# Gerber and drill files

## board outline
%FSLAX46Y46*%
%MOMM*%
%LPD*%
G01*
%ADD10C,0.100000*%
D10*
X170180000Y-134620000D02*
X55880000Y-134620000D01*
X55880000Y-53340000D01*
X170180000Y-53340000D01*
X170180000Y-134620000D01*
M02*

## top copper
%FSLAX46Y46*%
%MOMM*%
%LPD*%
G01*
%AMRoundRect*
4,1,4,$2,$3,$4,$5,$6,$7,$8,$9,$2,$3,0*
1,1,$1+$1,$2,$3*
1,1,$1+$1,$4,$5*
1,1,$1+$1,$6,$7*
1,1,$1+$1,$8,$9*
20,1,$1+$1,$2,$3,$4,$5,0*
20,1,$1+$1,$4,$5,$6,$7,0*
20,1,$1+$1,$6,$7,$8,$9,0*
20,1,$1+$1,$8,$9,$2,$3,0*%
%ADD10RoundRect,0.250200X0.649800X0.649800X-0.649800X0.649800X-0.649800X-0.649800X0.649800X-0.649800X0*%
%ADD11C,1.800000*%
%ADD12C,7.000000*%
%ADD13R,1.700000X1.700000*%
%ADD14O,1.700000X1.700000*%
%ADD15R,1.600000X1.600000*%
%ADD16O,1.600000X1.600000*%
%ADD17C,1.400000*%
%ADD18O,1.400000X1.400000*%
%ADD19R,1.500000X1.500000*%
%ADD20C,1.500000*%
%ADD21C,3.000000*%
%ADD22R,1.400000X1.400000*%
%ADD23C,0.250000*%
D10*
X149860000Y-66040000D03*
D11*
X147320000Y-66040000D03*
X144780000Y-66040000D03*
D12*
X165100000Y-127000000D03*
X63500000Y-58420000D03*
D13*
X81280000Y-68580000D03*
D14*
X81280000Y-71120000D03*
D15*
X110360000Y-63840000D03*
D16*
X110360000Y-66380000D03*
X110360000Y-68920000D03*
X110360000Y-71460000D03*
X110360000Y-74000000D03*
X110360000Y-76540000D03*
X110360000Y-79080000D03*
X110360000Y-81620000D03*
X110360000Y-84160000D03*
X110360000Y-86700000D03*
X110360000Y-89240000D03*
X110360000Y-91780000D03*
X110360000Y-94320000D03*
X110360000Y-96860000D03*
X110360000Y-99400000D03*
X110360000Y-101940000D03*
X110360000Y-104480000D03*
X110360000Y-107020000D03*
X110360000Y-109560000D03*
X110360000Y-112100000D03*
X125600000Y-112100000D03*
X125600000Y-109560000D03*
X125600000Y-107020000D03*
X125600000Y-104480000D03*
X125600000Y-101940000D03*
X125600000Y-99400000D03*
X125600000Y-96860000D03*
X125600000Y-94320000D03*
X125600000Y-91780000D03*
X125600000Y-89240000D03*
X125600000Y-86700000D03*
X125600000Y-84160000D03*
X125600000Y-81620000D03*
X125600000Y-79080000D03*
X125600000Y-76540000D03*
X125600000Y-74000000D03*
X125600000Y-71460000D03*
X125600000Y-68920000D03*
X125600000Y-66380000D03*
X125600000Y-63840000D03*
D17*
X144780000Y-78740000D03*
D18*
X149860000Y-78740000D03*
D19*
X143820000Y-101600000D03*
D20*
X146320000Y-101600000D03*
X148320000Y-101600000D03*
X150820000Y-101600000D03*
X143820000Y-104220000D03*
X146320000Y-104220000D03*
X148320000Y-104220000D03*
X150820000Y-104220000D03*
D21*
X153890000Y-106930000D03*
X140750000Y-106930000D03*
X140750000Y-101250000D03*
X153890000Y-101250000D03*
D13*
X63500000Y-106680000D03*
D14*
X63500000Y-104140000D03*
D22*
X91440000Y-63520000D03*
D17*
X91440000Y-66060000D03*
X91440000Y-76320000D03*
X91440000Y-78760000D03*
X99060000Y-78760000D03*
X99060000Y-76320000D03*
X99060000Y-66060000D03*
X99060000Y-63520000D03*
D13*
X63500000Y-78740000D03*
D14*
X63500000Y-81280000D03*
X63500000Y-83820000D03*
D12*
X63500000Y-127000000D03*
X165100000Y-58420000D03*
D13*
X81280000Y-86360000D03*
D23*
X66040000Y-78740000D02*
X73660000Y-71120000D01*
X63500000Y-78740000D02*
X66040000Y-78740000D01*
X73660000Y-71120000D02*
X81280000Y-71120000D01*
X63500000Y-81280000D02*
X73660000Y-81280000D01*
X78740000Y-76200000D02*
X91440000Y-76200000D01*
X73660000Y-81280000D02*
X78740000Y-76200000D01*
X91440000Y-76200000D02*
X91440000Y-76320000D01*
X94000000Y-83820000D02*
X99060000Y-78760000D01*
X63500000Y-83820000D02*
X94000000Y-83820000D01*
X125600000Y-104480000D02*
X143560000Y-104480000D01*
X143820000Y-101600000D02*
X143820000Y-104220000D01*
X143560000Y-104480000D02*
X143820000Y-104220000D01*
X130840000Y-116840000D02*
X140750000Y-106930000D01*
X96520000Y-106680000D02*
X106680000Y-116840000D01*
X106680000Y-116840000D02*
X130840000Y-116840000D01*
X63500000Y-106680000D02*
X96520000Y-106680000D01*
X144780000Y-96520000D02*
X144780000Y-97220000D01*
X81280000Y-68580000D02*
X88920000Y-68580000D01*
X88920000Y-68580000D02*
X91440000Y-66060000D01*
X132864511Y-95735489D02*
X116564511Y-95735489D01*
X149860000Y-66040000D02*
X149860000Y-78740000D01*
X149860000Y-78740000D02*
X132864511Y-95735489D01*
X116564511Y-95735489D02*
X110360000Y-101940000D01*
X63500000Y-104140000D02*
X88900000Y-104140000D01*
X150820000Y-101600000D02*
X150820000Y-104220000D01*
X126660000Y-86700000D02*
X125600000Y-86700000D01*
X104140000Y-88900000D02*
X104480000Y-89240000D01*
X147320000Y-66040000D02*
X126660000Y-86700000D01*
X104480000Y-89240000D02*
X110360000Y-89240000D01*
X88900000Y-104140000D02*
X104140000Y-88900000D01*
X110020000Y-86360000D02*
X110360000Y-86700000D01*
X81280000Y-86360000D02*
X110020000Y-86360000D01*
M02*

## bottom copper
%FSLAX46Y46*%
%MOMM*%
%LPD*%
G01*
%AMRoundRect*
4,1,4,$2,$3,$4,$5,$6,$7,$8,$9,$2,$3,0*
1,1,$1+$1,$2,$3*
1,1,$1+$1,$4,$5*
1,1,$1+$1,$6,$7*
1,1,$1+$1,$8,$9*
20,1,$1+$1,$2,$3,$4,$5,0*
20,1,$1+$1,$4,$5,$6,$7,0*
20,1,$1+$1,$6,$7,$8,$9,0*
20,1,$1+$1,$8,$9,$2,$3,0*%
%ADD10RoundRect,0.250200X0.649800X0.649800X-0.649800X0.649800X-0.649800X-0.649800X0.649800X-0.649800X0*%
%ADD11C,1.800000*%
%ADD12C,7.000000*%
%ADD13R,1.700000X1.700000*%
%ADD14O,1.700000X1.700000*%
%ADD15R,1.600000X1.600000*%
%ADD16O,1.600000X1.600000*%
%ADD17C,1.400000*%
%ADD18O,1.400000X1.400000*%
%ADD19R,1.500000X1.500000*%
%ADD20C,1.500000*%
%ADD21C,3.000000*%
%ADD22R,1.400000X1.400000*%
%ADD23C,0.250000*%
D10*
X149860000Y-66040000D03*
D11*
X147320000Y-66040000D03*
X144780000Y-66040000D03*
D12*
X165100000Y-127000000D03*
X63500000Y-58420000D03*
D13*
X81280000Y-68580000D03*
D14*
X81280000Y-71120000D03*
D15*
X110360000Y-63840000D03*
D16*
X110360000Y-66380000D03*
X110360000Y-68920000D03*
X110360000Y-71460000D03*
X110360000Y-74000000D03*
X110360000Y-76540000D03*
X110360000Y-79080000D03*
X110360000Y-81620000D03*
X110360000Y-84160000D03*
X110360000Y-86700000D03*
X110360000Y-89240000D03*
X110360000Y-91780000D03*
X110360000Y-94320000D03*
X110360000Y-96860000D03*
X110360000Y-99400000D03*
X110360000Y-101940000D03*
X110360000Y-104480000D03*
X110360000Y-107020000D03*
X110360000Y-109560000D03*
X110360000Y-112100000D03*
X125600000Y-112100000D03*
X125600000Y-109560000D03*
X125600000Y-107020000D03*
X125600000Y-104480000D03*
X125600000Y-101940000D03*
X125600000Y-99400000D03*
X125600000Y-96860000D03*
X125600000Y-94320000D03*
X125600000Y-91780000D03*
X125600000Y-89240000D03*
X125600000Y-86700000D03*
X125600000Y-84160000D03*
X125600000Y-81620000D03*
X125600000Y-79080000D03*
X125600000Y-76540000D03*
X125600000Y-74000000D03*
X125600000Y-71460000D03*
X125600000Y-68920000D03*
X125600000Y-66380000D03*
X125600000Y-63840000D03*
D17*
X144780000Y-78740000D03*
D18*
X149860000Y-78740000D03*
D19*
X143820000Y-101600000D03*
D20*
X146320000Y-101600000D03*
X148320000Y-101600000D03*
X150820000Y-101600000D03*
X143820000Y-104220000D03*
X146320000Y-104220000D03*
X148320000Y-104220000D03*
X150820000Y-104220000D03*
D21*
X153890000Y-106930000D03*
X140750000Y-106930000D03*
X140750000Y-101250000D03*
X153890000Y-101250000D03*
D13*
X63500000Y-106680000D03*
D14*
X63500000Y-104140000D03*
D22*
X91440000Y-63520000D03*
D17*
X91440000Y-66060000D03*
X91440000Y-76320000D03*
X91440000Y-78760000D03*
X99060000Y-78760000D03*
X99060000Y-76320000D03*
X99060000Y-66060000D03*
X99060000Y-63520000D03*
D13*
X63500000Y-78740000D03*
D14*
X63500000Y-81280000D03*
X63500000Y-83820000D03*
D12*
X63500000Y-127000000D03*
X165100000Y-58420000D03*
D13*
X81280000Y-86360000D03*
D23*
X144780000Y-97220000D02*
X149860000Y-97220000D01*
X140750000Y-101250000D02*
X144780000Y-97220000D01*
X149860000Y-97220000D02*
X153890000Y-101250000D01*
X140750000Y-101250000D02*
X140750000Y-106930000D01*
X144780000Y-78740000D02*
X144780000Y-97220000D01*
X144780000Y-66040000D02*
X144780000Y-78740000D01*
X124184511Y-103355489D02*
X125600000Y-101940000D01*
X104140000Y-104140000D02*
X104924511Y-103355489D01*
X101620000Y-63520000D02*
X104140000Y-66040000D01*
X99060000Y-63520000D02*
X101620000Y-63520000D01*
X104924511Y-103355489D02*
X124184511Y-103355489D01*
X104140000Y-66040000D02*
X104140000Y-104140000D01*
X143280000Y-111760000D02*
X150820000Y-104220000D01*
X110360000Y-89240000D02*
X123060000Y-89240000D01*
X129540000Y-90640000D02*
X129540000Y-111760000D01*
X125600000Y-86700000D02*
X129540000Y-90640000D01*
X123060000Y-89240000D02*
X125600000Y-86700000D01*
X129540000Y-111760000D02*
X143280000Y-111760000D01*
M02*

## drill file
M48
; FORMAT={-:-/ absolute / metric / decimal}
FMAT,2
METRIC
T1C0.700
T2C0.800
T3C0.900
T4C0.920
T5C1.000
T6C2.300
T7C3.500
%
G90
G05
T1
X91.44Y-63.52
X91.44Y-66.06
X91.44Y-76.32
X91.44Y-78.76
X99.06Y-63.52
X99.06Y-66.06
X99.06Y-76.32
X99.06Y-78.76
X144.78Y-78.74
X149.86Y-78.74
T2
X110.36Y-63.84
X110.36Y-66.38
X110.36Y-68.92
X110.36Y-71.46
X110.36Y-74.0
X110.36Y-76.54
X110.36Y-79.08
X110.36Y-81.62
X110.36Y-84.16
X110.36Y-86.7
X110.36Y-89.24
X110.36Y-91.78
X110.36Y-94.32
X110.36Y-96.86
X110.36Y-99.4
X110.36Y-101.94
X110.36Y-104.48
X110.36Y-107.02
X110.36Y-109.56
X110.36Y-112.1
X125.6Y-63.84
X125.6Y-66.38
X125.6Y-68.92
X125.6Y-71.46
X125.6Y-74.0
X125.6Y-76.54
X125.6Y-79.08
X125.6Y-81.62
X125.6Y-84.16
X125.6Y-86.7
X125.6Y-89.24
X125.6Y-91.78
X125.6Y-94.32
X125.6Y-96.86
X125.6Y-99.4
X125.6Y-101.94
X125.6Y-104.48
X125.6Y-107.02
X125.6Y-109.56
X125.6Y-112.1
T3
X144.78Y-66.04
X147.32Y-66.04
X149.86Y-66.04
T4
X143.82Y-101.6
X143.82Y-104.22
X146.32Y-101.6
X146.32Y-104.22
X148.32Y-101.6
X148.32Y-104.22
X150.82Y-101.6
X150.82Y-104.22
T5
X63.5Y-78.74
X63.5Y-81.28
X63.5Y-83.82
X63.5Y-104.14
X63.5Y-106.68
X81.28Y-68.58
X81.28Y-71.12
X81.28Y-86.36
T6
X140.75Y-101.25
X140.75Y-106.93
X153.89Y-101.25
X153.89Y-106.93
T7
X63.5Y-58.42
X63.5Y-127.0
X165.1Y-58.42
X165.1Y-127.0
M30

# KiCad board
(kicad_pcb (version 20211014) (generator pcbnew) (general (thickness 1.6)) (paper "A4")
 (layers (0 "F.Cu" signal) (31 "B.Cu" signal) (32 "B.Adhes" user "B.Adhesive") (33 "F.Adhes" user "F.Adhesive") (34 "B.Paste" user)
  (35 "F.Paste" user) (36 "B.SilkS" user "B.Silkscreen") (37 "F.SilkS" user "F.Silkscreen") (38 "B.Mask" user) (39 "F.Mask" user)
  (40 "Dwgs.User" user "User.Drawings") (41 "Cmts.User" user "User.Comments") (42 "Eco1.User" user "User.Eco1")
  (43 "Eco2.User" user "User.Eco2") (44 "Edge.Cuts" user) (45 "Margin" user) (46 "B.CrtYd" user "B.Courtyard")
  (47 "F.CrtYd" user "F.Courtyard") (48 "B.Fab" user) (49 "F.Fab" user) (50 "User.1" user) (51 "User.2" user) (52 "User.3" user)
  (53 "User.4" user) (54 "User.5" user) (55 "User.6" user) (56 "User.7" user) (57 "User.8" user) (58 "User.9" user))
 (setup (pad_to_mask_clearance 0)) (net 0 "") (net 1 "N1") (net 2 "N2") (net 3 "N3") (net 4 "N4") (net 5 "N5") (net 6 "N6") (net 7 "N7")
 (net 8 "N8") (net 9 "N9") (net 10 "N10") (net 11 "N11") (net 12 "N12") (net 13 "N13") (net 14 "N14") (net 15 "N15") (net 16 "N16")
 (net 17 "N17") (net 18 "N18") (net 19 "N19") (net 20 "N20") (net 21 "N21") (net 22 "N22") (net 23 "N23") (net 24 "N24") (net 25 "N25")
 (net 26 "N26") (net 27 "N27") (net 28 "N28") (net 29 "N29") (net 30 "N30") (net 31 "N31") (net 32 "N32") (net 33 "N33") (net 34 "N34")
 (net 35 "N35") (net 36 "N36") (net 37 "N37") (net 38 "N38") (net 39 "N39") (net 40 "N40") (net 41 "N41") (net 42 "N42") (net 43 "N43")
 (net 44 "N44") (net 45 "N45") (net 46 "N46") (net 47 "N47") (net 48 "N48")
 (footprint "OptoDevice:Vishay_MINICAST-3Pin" (layer "F.Cu") (at 149.86 66.04 180)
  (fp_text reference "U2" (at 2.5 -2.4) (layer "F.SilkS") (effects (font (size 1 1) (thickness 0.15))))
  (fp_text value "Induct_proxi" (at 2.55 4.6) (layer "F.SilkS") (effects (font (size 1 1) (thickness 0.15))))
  (pad "1" thru_hole roundrect (at 0 0 180) (size 1.8 1.8) (drill 0.9) (layers *.Cu *.Mask) (roundrect_rratio 0.139) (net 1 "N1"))
  (pad "2" thru_hole circle (at 2.54 0 180) (size 1.8 1.8) (drill 0.9) (layers *.Cu *.Mask) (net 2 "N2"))
  (pad "3" thru_hole circle (at 5.08 0 180) (size 1.8 1.8) (drill 0.9) (layers *.Cu *.Mask) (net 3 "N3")))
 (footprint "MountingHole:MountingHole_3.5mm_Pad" (layer "F.Cu") (at 165.1 127)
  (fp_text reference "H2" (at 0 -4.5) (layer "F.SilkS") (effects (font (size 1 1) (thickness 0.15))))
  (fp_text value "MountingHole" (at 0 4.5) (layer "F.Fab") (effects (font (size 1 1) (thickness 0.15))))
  (pad "1" thru_hole circle (at 0 0) (size 7 7) (drill 3.5) (layers *.Cu *.Mask)))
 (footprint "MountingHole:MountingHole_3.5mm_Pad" (layer "F.Cu") (at 63.5 58.42)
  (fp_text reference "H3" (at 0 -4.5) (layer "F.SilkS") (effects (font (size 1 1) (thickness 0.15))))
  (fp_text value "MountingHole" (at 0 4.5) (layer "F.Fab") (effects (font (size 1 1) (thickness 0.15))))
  (pad "1" thru_hole circle (at 0 0) (size 7 7) (drill 3.5) (layers *.Cu *.Mask)))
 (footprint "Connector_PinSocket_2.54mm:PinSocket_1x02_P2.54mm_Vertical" (layer "F.Cu") (at 81.28 68.58)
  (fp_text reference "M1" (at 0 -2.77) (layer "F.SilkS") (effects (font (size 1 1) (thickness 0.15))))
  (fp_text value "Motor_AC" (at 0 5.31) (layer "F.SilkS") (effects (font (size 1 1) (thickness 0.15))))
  (pad "1" thru_hole rect (at 0 0) (size 1.7 1.7) (drill 1) (layers *.Cu *.Mask) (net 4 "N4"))
  (pad "2" thru_hole oval (at 0 2.54) (size 1.7 1.7) (drill 1) (layers *.Cu *.Mask) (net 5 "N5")))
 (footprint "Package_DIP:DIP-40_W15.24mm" (layer "F.Cu") (at 110.36 63.84)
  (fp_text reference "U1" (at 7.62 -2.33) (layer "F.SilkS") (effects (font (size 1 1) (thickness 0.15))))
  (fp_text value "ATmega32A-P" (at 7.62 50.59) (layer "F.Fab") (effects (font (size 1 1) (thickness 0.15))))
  (pad "1" thru_hole rect (at 0 0) (size 1.6 1.6) (drill 0.8) (layers *.Cu *.Mask) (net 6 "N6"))
  (pad "2" thru_hole oval (at 0 2.54) (size 1.6 1.6) (drill 0.8) (layers *.Cu *.Mask) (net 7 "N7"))
  (pad "3" thru_hole oval (at 0 5.08) (size 1.6 1.6) (drill 0.8) (layers *.Cu *.Mask) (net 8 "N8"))
  (pad "4" thru_hole oval (at 0 7.62) (size 1.6 1.6) (drill 0.8) (layers *.Cu *.Mask) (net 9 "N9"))
  (pad "5" thru_hole oval (at 0 10.16) (size 1.6 1.6) (drill 0.8) (layers *.Cu *.Mask) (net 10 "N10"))
  (pad "6" thru_hole oval (at 0 12.7) (size 1.6 1.6) (drill 0.8) (layers *.Cu *.Mask) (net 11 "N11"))
  (pad "7" thru_hole oval (at 0 15.24) (size 1.6 1.6) (drill 0.8) (layers *.Cu *.Mask) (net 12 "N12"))
  (pad "8" thru_hole oval (at 0 17.78) (size 1.6 1.6) (drill 0.8) (layers *.Cu *.Mask) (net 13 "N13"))
  (pad "9" thru_hole oval (at 0 20.32) (size 1.6 1.6) (drill 0.8) (layers *.Cu *.Mask) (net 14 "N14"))
  (pad "10" thru_hole oval (at 0 22.86) (size 1.6 1.6) (drill 0.8) (layers *.Cu *.Mask) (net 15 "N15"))
  (pad "11" thru_hole oval (at 0 25.4) (size 1.6 1.6) (drill 0.8) (layers *.Cu *.Mask) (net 2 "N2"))
  (pad "12" thru_hole oval (at 0 27.94) (size 1.6 1.6) (drill 0.8) (layers *.Cu *.Mask) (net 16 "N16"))
  (pad "13" thru_hole oval (at 0 30.48) (size 1.6 1.6) (drill 0.8) (layers *.Cu *.Mask) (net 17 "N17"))
  (pad "14" thru_hole oval (at 0 33.02) (size 1.6 1.6) (drill 0.8) (layers *.Cu *.Mask) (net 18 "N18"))
  (pad "15" thru_hole oval (at 0 35.56) (size 1.6 1.6) (drill 0.8) (layers *.Cu *.Mask) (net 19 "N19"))
  (pad "16" thru_hole oval (at 0 38.1) (size 1.6 1.6) (drill 0.8) (layers *.Cu *.Mask) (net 1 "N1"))
  (pad "17" thru_hole oval (at 0 40.64) (size 1.6 1.6) (drill 0.8) (layers *.Cu *.Mask) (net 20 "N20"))
  (pad "18" thru_hole oval (at 0 43.18) (size 1.6 1.6) (drill 0.8) (layers *.Cu *.Mask) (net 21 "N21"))
  (pad "19" thru_hole oval (at 0 45.72) (size 1.6 1.6) (drill 0.8) (layers *.Cu *.Mask) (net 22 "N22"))
  (pad "20" thru_hole oval (at 0 48.26) (size 1.6 1.6) (drill 0.8) (layers *.Cu *.Mask) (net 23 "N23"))
  (pad "21" thru_hole oval (at 15.24 48.26) (size 1.6 1.6) (drill 0.8) (layers *.Cu *.Mask) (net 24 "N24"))
  (pad "22" thru_hole oval (at 15.24 45.72) (size 1.6 1.6) (drill 0.8) (layers *.Cu *.Mask) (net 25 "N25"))
  (pad "23" thru_hole oval (at 15.24 43.18) (size 1.6 1.6) (drill 0.8) (layers *.Cu *.Mask) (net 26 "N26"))
  (pad "24" thru_hole oval (at 15.24 40.64) (size 1.6 1.6) (drill 0.8) (layers *.Cu *.Mask) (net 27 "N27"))
  (pad "25" thru_hole oval (at 15.24 38.1) (size 1.6 1.6) (drill 0.8) (layers *.Cu *.Mask) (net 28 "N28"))
  (pad "26" thru_hole oval (at 15.24 35.56) (size 1.6 1.6) (drill 0.8) (layers *.Cu *.Mask) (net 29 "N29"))
  (pad "27" thru_hole oval (at 15.24 33.02) (size 1.6 1.6) (drill 0.8) (layers *.Cu *.Mask) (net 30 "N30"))
  (pad "28" thru_hole oval (at 15.24 30.48) (size 1.6 1.6) (drill 0.8) (layers *.Cu *.Mask) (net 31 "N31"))
  (pad "29" thru_hole oval (at 15.24 27.94) (size 1.6 1.6) (drill 0.8) (layers *.Cu *.Mask) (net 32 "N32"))
  (pad "30" thru_hole oval (at 15.24 25.4) (size 1.6 1.6) (drill 0.8) (layers *.Cu *.Mask) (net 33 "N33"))
  (pad "31" thru_hole oval (at 15.24 22.86) (size 1.6 1.6) (drill 0.8) (layers *.Cu *.Mask) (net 2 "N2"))
  (pad "32" thru_hole oval (at 15.24 20.32) (size 1.6 1.6) (drill 0.8) (layers *.Cu *.Mask) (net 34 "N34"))
  (pad "33" thru_hole oval (at 15.24 17.78) (size 1.6 1.6) (drill 0.8) (layers *.Cu *.Mask) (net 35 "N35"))
  (pad "34" thru_hole oval (at 15.24 15.24) (size 1.6 1.6) (drill 0.8) (layers *.Cu *.Mask) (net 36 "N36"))
  (pad "35" thru_hole oval (at 15.24 12.7) (size 1.6 1.6) (drill 0.8) (layers *.Cu *.Mask) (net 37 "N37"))
  (pad "36" thru_hole oval (at 15.24 10.16) (size 1.6 1.6) (drill 0.8) (layers *.Cu *.Mask) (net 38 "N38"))
  (pad "37" thru_hole oval (at 15.24 7.62) (size 1.6 1.6) (drill 0.8) (layers *.Cu *.Mask) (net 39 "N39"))
  (pad "38" thru_hole oval (at 15.24 5.08) (size 1.6 1.6) (drill 0.8) (layers *.Cu *.Mask) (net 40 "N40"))
  (pad "39" thru_hole oval (at 15.24 2.54) (size 1.6 1.6) (drill 0.8) (layers *.Cu *.Mask) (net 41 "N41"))
  (pad "40" thru_hole oval (at 15.24 0) (size 1.6 1.6) (drill 0.8) (layers *.Cu *.Mask) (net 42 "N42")))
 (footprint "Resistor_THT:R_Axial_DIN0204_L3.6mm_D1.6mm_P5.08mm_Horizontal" (layer "F.Cu") (at 144.78 78.74)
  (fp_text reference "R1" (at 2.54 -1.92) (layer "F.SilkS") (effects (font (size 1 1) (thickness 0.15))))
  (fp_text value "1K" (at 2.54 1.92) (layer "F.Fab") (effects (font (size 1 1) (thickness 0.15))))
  (pad "1" thru_hole circle (at 0 0) (size 1.4 1.4) (drill 0.7) (layers *.Cu *.Mask) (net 3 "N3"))
  (pad "2" thru_hole oval (at 5.08 0) (size 1.4 1.4) (drill 0.7) (layers *.Cu *.Mask) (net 1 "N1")))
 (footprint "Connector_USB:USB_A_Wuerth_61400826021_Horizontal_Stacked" (layer "F.Cu") (at 143.82 101.6)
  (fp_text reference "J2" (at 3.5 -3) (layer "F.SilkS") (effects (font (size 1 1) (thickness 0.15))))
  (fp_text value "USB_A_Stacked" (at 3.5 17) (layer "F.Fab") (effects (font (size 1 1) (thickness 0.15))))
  (pad "1" thru_hole rect (at 0 0) (size 1.5 1.5) (drill 0.92) (layers *.Cu *.Mask) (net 27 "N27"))
  (pad "2" thru_hole circle (at 2.5 0) (size 1.5 1.5) (drill 0.92) (layers *.Cu *.Mask) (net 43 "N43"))
  (pad "3" thru_hole circle (at 4.5 0) (size 1.5 1.5) (drill 0.92) (layers *.Cu *.Mask) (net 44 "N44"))
  (pad "4" thru_hole circle (at 7 0) (size 1.5 1.5) (drill 0.92) (layers *.Cu *.Mask) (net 2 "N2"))
  (pad "5" thru_hole circle (at 0 2.62) (size 1.5 1.5) (drill 0.92) (layers *.Cu *.Mask) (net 27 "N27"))
  (pad "6" thru_hole circle (at 2.5 2.62) (size 1.5 1.5) (drill 0.92) (layers *.Cu *.Mask) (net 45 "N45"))
  (pad "7" thru_hole circle (at 4.5 2.62) (size 1.5 1.5) (drill 0.92) (layers *.Cu *.Mask) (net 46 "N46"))
  (pad "8" thru_hole circle (at 7 2.62) (size 1.5 1.5) (drill 0.92) (layers *.Cu *.Mask) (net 2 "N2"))
  (pad "9" thru_hole circle (at 10.07 5.33) (size 3 3) (drill 2.3) (layers *.Cu *.Mask) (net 3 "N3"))
  (pad "9" thru_hole circle (at -3.07 5.33) (size 3 3) (drill 2.3) (layers *.Cu *.Mask) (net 3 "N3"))
  (pad "9" thru_hole circle (at -3.07 -0.35) (size 3 3) (drill 2.3) (layers *.Cu *.Mask) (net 3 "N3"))
  (pad "9" thru_hole circle (at 10.07 -0.35) (size 3 3) (drill 2.3) (layers *.Cu *.Mask) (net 3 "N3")))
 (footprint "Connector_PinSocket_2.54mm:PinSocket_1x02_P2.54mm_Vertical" (layer "F.Cu") (at 63.5 106.68 180)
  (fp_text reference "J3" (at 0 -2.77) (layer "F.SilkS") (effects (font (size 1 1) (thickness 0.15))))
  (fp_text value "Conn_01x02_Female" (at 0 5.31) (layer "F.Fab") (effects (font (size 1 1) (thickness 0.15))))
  (pad "1" thru_hole rect (at 0 0 180) (size 1.7 1.7) (drill 1) (layers *.Cu *.Mask) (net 3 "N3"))
  (pad "2" thru_hole oval (at 0 2.54 180) (size 1.7 1.7) (drill 1) (layers *.Cu *.Mask) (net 2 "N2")))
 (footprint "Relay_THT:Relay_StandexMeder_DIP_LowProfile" (layer "F.Cu") (at 91.44 63.52)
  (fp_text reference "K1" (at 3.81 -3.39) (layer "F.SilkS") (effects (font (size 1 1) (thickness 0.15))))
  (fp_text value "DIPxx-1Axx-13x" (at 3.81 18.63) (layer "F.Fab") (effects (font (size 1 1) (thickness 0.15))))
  (pad "1" thru_hole rect (at 0 0) (size 1.4 1.4) (drill 0.7) (layers *.Cu *.Mask))
  (pad "2" thru_hole circle (at 0 2.54) (size 1.4 1.4) (drill 0.7) (layers *.Cu *.Mask) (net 4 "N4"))
  (pad "6" thru_hole circle (at 0 12.8) (size 1.4 1.4) (drill 0.7) (layers *.Cu *.Mask) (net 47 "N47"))
  (pad "7" thru_hole circle (at 0 15.24) (size 1.4 1.4) (drill 0.7) (layers *.Cu *.Mask))
  (pad "8" thru_hole circle (at 7.62 15.24) (size 1.4 1.4) (drill 0.7) (layers *.Cu *.Mask) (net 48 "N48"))
  (pad "9" thru_hole circle (at 7.62 12.8) (size 1.4 1.4) (drill 0.7) (layers *.Cu *.Mask))
  (pad "13" thru_hole circle (at 7.62 2.54) (size 1.4 1.4) (drill 0.7) (layers *.Cu *.Mask))
  (pad "14" thru_hole circle (at 7.62 0) (size 1.4 1.4) (drill 0.7) (layers *.Cu *.Mask) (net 28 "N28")))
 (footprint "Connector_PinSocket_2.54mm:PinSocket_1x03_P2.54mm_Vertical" (layer "F.Cu") (at 63.5 78.74)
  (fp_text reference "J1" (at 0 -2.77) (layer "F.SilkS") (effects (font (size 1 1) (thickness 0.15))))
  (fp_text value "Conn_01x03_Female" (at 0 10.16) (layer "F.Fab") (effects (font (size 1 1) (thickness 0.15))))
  (pad "1" thru_hole rect (at 0 0) (size 1.7 1.7) (drill 1) (layers *.Cu *.Mask) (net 5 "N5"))
  (pad "2" thru_hole oval (at 0 2.54) (size 1.7 1.7) (drill 1) (layers *.Cu *.Mask) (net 47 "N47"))
  (pad "3" thru_hole oval (at 0 5.08) (size 1.7 1.7) (drill 1) (layers *.Cu *.Mask) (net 48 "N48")))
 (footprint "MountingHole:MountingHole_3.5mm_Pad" (layer "F.Cu") (at 63.5 127)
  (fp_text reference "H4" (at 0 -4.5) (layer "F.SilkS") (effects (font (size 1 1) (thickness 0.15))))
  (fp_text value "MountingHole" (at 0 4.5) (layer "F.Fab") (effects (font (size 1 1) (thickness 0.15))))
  (pad "1" thru_hole circle (at 0 0) (size 7 7) (drill 3.5) (layers *.Cu *.Mask)))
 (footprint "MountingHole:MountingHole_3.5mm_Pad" (layer "F.Cu") (at 165.1 58.42)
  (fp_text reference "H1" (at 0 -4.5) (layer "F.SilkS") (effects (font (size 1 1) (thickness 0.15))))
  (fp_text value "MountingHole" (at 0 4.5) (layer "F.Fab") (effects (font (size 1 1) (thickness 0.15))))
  (pad "1" thru_hole circle (at 0 0) (size 7 7) (drill 3.5) (layers *.Cu *.Mask)))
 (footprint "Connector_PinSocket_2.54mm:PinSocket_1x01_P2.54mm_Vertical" (layer "F.Cu") (at 81.28 86.36)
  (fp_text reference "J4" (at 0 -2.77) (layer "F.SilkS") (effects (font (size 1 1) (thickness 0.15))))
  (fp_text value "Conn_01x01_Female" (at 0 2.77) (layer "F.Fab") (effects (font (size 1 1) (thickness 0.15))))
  (pad "1" thru_hole rect (at 0 0) (size 1.7 1.7) (drill 1) (layers *.Cu *.Mask) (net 15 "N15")))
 (gr_poly (pts (xy 170.18 134.62) (xy 55.88 134.62) (xy 55.88 53.34) (xy 170.18 53.34)) (layer "Edge.Cuts") (width 0.1) (fill none))
 (segment (start 66.04 78.74) (end 73.66 71.12) (width 0.25) (layer "F.Cu") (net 5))
 (segment (start 63.5 78.74) (end 66.04 78.74) (width 0.25) (layer "F.Cu") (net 5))
 (segment (start 73.66 71.12) (end 81.28 71.12) (width 0.25) (layer "F.Cu") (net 5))
 (segment (start 63.5 81.28) (end 73.66 81.28) (width 0.25) (layer "F.Cu") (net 47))
 (segment (start 78.74 76.2) (end 91.44 76.2) (width 0.25) (layer "F.Cu") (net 47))
 (segment (start 73.66 81.28) (end 78.74 76.2) (width 0.25) (layer "F.Cu") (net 47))
 (segment (start 91.44 76.2) (end 91.44 76.32) (width 0.25) (layer "F.Cu") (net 47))
 (segment (start 94 83.82) (end 99.06 78.76) (width 0.25) (layer "F.Cu") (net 48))
 (segment (start 63.5 83.82) (end 94 83.82) (width 0.25) (layer "F.Cu") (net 48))
 (segment (start 125.6 104.48) (end 143.56 104.48) (width 0.25) (layer "F.Cu") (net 27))
 (segment (start 143.82 101.6) (end 143.82 104.22) (width 0.25) (layer "F.Cu") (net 27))
 (segment (start 143.56 104.48) (end 143.82 104.22) (width 0.25) (layer "F.Cu") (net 27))
 (segment (start 130.84 116.84) (end 140.75 106.93) (width 0.25) (layer "F.Cu") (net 3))
 (segment (start 96.52 106.68) (end 106.68 116.84) (width 0.25) (layer "F.Cu") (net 3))
 (segment (start 106.68 116.84) (end 130.84 116.84) (width 0.25) (layer "F.Cu") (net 3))
 (segment (start 63.5 106.68) (end 96.52 106.68) (width 0.25) (layer "F.Cu") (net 3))
 (segment (start 144.78 96.52) (end 144.78 97.22) (width 0.25) (layer "F.Cu") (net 3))
 (segment (start 144.78 97.22) (end 149.86 97.22) (width 0.25) (layer "B.Cu") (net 3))
 (segment (start 140.75 101.25) (end 144.78 97.22) (width 0.25) (layer "B.Cu") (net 3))
 (segment (start 149.86 97.22) (end 153.89 101.25) (width 0.25) (layer "B.Cu") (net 3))
 (segment (start 140.75 101.25) (end 140.75 106.93) (width 0.25) (layer "B.Cu") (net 3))
 (segment (start 144.78 78.74) (end 144.78 97.22) (width 0.25) (layer "B.Cu") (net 3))
 (segment (start 144.78 66.04) (end 144.78 78.74) (width 0.25) (layer "B.Cu") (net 3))
 (segment (start 81.28 68.58) (end 88.92 68.58) (width 0.25) (layer "F.Cu") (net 4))
 (segment (start 88.92 68.58) (end 91.44 66.06) (width 0.25) (layer "F.Cu") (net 4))
 (segment (start 124.184511 103.355489) (end 125.6 101.94) (width 0.25) (layer "B.Cu") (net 28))
 (segment (start 104.14 104.14) (end 104.924511 103.355489) (width 0.25) (layer "B.Cu") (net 28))
 (segment (start 101.62 63.52) (end 104.14 66.04) (width 0.25) (layer "B.Cu") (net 28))
 (segment (start 99.06 63.52) (end 101.62 63.52) (width 0.25) (layer "B.Cu") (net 28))
 (segment (start 104.924511 103.355489) (end 124.184511 103.355489) (width 0.25) (layer "B.Cu") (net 28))
 (segment (start 104.14 66.04) (end 104.14 104.14) (width 0.25) (layer "B.Cu") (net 28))
 (segment (start 132.864511 95.735489) (end 116.564511 95.735489) (width 0.25) (layer "F.Cu") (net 1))
 (segment (start 149.86 66.04) (end 149.86 78.74) (width 0.25) (layer "F.Cu") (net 1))
 (segment (start 149.86 78.74) (end 132.864511 95.735489) (width 0.25) (layer "F.Cu") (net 1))
 (segment (start 116.564511 95.735489) (end 110.36 101.94) (width 0.25) (layer "F.Cu") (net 1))
 (segment (start 63.5 104.14) (end 88.9 104.14) (width 0.25) (layer "F.Cu") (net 2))
 (segment (start 150.82 101.6) (end 150.82 104.22) (width 0.25) (layer "F.Cu") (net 2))
 (segment (start 126.66 86.7) (end 125.6 86.7) (width 0.25) (layer "F.Cu") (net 2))
 (segment (start 104.14 88.9) (end 104.48 89.24) (width 0.25) (layer "F.Cu") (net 2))
 (segment (start 147.32 66.04) (end 126.66 86.7) (width 0.25) (layer "F.Cu") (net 2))
 (segment (start 104.48 89.24) (end 110.36 89.24) (width 0.25) (layer "F.Cu") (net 2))
 (segment (start 88.9 104.14) (end 104.14 88.9) (width 0.25) (layer "F.Cu") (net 2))
 (segment (start 143.28 111.76) (end 150.82 104.22) (width 0.25) (layer "B.Cu") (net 2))
 (segment (start 110.36 89.24) (end 123.06 89.24) (width 0.25) (layer "B.Cu") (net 2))
 (segment (start 129.54 90.64) (end 129.54 111.76) (width 0.25) (layer "B.Cu") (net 2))
 (segment (start 125.6 86.7) (end 129.54 90.64) (width 0.25) (layer "B.Cu") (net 2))
 (segment (start 123.06 89.24) (end 125.6 86.7) (width 0.25) (layer "B.Cu") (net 2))
 (segment (start 129.54 111.76) (end 143.28 111.76) (width 0.25) (layer "B.Cu") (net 2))
 (segment (start 110.02 86.36) (end 110.36 86.7) (width 0.25) (layer "F.Cu") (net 15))
 (segment (start 81.28 86.36) (end 110.02 86.36) (width 0.25) (layer "F.Cu") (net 15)))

